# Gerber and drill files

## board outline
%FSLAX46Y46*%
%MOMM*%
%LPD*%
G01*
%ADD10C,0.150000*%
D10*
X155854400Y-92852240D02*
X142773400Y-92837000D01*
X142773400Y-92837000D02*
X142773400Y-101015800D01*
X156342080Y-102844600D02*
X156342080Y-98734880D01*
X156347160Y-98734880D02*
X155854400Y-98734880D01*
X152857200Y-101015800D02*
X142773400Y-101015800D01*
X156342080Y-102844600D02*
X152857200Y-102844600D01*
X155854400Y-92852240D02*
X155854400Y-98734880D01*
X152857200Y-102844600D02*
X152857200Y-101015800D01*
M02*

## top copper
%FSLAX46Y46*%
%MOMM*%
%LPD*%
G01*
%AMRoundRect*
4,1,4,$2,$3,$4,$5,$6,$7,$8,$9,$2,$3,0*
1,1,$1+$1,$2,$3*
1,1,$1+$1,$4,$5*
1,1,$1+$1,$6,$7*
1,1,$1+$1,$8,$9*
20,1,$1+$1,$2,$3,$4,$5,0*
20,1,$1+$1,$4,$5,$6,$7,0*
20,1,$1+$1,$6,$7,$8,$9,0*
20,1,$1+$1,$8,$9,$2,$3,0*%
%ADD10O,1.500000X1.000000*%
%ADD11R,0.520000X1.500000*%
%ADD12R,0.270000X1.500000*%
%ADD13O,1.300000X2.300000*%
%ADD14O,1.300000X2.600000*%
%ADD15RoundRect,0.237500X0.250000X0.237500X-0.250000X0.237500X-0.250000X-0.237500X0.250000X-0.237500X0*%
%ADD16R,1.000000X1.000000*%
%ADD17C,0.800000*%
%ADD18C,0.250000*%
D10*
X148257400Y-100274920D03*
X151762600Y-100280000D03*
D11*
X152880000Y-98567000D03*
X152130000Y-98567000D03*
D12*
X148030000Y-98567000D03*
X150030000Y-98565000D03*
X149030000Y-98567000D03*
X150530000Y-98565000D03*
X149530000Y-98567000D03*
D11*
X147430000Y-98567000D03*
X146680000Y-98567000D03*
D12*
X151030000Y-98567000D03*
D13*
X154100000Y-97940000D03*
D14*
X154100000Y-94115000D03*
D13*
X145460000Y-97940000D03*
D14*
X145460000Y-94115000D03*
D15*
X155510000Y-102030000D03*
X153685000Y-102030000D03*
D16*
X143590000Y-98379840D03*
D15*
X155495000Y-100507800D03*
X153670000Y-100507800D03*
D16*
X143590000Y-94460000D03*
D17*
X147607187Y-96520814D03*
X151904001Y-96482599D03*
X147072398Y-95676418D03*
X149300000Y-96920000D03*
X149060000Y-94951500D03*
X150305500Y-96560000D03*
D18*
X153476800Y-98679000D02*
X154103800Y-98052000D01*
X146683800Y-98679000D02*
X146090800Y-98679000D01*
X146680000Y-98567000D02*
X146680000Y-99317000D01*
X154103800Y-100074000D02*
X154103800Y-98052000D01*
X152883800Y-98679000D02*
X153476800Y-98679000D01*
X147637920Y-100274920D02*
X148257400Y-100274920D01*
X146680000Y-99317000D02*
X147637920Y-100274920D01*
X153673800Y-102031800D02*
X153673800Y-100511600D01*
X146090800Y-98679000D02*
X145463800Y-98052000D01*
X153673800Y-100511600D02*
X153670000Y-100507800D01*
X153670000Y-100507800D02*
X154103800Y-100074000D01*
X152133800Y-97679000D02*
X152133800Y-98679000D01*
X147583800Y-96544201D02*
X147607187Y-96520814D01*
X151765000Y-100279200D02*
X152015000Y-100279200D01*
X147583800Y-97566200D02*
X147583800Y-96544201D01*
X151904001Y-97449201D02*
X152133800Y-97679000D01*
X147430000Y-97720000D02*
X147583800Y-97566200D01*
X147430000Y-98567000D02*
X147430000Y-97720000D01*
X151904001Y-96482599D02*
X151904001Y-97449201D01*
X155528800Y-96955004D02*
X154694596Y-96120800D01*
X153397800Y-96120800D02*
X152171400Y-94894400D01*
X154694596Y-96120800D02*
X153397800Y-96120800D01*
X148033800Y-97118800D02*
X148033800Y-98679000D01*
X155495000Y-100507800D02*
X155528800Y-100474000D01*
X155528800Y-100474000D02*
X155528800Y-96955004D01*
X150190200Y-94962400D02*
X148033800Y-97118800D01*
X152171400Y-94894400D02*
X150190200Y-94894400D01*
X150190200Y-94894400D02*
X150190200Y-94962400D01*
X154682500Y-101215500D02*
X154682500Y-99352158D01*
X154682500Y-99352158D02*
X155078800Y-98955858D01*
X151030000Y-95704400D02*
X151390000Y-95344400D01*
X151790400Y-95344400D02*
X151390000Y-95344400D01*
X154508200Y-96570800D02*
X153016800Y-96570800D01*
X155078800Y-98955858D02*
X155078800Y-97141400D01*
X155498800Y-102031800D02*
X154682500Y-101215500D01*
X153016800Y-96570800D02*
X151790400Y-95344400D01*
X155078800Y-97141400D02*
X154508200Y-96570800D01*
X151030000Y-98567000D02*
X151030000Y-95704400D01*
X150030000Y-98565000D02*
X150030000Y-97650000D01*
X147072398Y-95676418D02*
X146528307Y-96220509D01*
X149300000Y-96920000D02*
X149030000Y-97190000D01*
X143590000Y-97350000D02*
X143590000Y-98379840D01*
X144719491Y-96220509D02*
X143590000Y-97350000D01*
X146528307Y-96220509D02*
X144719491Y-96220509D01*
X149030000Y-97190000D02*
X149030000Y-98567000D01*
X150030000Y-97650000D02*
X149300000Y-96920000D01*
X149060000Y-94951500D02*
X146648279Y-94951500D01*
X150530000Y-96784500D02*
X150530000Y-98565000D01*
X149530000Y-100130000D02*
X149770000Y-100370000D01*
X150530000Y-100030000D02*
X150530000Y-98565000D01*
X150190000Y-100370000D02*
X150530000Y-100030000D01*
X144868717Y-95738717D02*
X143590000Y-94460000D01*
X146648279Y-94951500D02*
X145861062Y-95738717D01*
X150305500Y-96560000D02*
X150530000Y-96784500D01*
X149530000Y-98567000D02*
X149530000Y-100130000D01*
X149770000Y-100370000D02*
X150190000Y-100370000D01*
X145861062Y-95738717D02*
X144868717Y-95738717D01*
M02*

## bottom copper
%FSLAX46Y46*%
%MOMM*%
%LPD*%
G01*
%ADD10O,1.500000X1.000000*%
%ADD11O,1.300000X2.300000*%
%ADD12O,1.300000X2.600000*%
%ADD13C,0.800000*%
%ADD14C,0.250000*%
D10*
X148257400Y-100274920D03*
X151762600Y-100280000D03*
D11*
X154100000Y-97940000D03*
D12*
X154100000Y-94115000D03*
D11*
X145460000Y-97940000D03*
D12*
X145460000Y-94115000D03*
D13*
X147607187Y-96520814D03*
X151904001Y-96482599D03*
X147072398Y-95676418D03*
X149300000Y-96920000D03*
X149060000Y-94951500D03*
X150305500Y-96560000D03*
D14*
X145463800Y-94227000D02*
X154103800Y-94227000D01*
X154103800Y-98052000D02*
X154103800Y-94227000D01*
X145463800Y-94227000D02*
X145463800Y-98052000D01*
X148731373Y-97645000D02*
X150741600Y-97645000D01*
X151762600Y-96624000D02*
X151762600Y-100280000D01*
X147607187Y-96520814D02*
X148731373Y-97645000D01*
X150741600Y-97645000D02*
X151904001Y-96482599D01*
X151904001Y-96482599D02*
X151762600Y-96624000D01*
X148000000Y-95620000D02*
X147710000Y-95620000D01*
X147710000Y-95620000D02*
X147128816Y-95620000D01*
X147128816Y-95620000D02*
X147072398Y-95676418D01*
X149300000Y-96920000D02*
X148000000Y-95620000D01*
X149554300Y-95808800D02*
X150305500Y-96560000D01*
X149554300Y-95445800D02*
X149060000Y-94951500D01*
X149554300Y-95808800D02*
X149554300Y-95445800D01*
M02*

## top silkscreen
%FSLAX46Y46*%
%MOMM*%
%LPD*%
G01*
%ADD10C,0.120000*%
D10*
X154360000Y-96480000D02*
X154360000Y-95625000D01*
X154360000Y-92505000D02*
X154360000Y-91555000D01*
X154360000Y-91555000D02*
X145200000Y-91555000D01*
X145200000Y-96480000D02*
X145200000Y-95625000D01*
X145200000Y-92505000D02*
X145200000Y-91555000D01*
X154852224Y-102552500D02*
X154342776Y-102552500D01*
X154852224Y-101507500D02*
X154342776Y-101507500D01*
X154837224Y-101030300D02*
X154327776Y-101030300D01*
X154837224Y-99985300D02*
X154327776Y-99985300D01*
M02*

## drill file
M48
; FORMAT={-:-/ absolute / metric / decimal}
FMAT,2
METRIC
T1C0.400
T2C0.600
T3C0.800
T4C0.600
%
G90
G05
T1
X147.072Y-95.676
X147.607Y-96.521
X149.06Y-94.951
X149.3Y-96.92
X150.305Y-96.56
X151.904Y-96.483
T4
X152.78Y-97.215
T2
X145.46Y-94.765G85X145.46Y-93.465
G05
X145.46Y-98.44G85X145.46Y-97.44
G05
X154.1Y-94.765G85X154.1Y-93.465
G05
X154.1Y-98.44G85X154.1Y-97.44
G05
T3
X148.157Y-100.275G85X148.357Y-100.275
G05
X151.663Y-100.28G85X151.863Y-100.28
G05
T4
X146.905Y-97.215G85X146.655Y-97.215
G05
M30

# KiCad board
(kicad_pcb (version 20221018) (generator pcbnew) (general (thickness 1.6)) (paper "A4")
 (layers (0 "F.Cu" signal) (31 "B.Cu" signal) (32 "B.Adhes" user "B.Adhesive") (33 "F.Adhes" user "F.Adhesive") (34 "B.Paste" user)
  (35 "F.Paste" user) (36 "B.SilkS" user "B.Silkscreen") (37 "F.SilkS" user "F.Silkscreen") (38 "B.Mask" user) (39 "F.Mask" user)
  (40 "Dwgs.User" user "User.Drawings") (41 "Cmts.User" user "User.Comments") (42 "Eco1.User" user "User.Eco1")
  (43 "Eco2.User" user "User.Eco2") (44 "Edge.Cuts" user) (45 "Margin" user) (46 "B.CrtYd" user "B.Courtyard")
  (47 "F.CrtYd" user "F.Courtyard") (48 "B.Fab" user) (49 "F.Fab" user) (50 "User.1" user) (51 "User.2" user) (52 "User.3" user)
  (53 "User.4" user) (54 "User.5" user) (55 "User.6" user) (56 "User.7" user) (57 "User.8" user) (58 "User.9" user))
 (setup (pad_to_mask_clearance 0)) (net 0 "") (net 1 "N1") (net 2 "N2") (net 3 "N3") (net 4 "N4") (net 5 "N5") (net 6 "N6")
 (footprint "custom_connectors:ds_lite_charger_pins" (layer "F.Cu") (at 150.01 100.28)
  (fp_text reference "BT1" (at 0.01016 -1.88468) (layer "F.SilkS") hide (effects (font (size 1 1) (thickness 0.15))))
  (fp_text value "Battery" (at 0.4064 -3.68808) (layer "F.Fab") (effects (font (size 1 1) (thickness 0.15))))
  (pad "1" thru_hole oval (at -1.7526 -0.00508 90) (size 1 1.5) (drill oval 0.8 1) (layers "*.Cu" "*.Mask") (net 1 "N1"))
  (pad "2" thru_hole oval (at 1.7526 0 90) (size 1 1.5) (drill oval 0.8 1) (layers "*.Cu" "*.Mask") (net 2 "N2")))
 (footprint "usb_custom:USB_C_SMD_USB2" (layer "F.Cu") (at 149.78 95.265 180)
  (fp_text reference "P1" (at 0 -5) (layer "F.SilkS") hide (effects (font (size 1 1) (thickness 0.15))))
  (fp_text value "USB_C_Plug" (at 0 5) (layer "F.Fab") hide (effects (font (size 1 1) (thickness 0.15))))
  (fp_line (start -4.58 -1.215) (end -4.58 -0.36) (stroke (width 0.12) (type solid)) (layer "F.SilkS"))
  (fp_line (start -4.58 2.76) (end -4.58 3.71) (stroke (width 0.12) (type solid)) (layer "F.SilkS"))
  (fp_line (start -4.58 3.71) (end 4.58 3.71) (stroke (width 0.12) (type solid)) (layer "F.SilkS"))
  (fp_line (start 4.58 -1.215) (end 4.58 -0.36) (stroke (width 0.12) (type solid)) (layer "F.SilkS"))
  (fp_line (start 4.58 2.76) (end 4.58 3.71) (stroke (width 0.12) (type solid)) (layer "F.SilkS"))
  (pad "" np_thru_hole circle (at -3 -1.95 180) (size 0.6 0.6) (drill 0.6) (layers "F&B.Cu" "*.Mask"))
  (pad "" np_thru_hole oval (at 3 -1.95 180) (size 0.85 0.6) (drill oval 0.85 0.6) (layers "F&B.Cu" "*.Mask"))
  (pad "A1" smd rect (at -3.1 -3.302 180) (size 0.52 1.5) (layers "F.Cu" "F.Paste" "F.Mask") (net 1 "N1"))
  (pad "A4" smd rect (at -2.35 -3.302 180) (size 0.52 1.5) (layers "F.Cu" "F.Paste" "F.Mask") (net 2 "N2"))
  (pad "A5" smd rect (at 1.75 -3.302 180) (size 0.27 1.5) (layers "F.Cu" "F.Paste" "F.Mask") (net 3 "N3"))
  (pad "A6" smd rect (at -0.25 -3.3 180) (size 0.27 1.5) (layers "F.Cu" "F.Paste" "F.Mask") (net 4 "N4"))
  (pad "A6" smd rect (at 0.75 -3.302 180) (size 0.27 1.5) (layers "F.Cu" "F.Paste" "F.Mask") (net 4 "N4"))
  (pad "A7" smd rect (at -0.75 -3.3 180) (size 0.27 1.5) (layers "F.Cu" "F.Paste" "F.Mask") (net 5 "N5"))
  (pad "A7" smd rect (at 0.25 -3.302 180) (size 0.27 1.5) (layers "F.Cu" "F.Paste" "F.Mask") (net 5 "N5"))
  (pad "A9" smd rect (at 2.35 -3.302 180) (size 0.52 1.5) (layers "F.Cu" "F.Paste" "F.Mask") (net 2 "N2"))
  (pad "A12" smd rect (at 3.1 -3.302 180) (size 0.52 1.5) (layers "F.Cu" "F.Paste" "F.Mask") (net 1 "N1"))
  (pad "B5" smd rect (at -1.25 -3.302 180) (size 0.27 1.5) (layers "F.Cu" "F.Paste" "F.Mask") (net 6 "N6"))
  (pad "S1" thru_hole oval (at -4.32 -2.675 180) (size 1.3 2.3) (drill oval 0.6 1.6) (layers "*.Cu" "*.Mask") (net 1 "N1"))
  (pad "S1" thru_hole oval (at -4.32 1.15 180) (size 1.3 2.6) (drill oval 0.6 1.9) (layers "*.Cu" "*.Mask") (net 1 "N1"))
  (pad "S1" thru_hole oval (at 4.32 -2.675 180) (size 1.3 2.3) (drill oval 0.6 1.6) (layers "*.Cu" "*.Mask") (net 1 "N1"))
  (pad "S1" thru_hole oval (at 4.32 1.15 180) (size 1.3 2.6) (drill oval 0.6 1.9) (layers "*.Cu" "*.Mask") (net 1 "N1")))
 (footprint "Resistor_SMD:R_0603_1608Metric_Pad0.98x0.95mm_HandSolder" (layer "F.Cu") (at 154.5975 102.03 180)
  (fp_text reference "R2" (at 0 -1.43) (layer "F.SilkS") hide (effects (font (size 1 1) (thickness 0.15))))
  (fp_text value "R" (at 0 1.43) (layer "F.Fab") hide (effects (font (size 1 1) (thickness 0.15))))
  (fp_line (start -0.254724 -0.5225) (end 0.254724 -0.5225) (stroke (width 0.12) (type solid)) (layer "F.SilkS"))
  (fp_line (start -0.254724 0.5225) (end 0.254724 0.5225) (stroke (width 0.12) (type solid)) (layer "F.SilkS"))
  (pad "1" smd roundrect (at -0.9125 0 180) (size 0.975 0.95) (layers "F.Cu" "F.Paste" "F.Mask") (roundrect_rratio 0.25) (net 6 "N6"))
  (pad "2" smd roundrect (at 0.9125 0 180) (size 0.975 0.95) (layers "F.Cu" "F.Paste" "F.Mask") (roundrect_rratio 0.25) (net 1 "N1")))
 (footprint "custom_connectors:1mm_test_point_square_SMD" (layer "F.Cu") (at 143.59 98.39)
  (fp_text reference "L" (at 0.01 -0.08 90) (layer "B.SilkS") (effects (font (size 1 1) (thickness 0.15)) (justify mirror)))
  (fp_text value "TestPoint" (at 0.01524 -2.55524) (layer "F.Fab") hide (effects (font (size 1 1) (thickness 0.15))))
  (pad "1" smd rect (at 0 -0.01016) (size 1 1) (layers "F.Cu" "F.Paste" "F.Mask") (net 4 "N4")))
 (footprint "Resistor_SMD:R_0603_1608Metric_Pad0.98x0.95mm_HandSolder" (layer "F.Cu") (at 154.5825 100.5078 180)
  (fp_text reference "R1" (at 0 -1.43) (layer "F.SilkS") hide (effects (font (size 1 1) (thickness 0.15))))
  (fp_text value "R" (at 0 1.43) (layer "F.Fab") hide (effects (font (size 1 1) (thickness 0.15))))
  (fp_line (start -0.254724 -0.5225) (end 0.254724 -0.5225) (stroke (width 0.12) (type solid)) (layer "F.SilkS"))
  (fp_line (start -0.254724 0.5225) (end 0.254724 0.5225) (stroke (width 0.12) (type solid)) (layer "F.SilkS"))
  (pad "1" smd roundrect (at -0.9125 0 180) (size 0.975 0.95) (layers "F.Cu" "F.Paste" "F.Mask") (roundrect_rratio 0.25) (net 3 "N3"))
  (pad "2" smd roundrect (at 0.9125 0 180) (size 0.975 0.95) (layers "F.Cu" "F.Paste" "F.Mask") (roundrect_rratio 0.25) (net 1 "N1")))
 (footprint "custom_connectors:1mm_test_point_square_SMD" (layer "F.Cu") (at 143.59 94.47016)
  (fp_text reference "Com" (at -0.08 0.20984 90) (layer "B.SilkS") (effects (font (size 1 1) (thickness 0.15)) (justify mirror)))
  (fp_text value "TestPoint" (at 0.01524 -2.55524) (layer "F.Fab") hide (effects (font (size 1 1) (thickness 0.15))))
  (pad "1" smd rect (at 0 -0.01016) (size 1 1) (layers "F.Cu" "F.Paste" "F.Mask") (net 5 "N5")))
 (gr_line (start 155.8544 92.85224) (end 142.7734 92.837) (stroke (width 0.15) (type solid)) (layer "Edge.Cuts"))
 (gr_line (start 142.7734 92.837) (end 142.7734 101.0158) (stroke (width 0.15) (type solid)) (layer "Edge.Cuts"))
 (gr_line (start 156.34208 102.8446) (end 156.34208 98.73488) (stroke (width 0.15) (type solid)) (layer "Edge.Cuts"))
 (gr_line (start 156.34716 98.73488) (end 155.8544 98.73488) (stroke (width 0.15) (type solid)) (layer "Edge.Cuts"))
 (gr_line (start 152.8572 101.0158) (end 142.7734 101.0158) (stroke (width 0.15) (type solid)) (layer "Edge.Cuts"))
 (gr_line (start 156.34208 102.8446) (end 152.8572 102.8446) (stroke (width 0.15) (type solid)) (layer "Edge.Cuts"))
 (gr_line (start 155.8544 92.85224) (end 155.8544 98.73488) (stroke (width 0.15) (type solid)) (layer "Edge.Cuts"))
 (gr_line (start 152.8572 102.8446) (end 152.8572 101.0158) (stroke (width 0.15) (type solid)) (layer "Edge.Cuts"))
 (segment (start 153.4768 98.679) (end 154.1038 98.052) (width 0.25) (layer "F.Cu") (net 1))
 (segment (start 146.6838 98.679) (end 146.0908 98.679) (width 0.25) (layer "F.Cu") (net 1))
 (segment (start 146.68 98.567) (end 146.68 99.317) (width 0.25) (layer "F.Cu") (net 1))
 (segment (start 154.1038 100.074) (end 154.1038 98.052) (width 0.25) (layer "F.Cu") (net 1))
 (segment (start 152.8838 98.679) (end 153.4768 98.679) (width 0.25) (layer "F.Cu") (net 1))
 (segment (start 147.63792 100.27492) (end 148.2574 100.27492) (width 0.25) (layer "F.Cu") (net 1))
 (segment (start 146.68 99.317) (end 147.63792 100.27492) (width 0.25) (layer "F.Cu") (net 1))
 (segment (start 153.6738 102.0318) (end 153.6738 100.5116) (width 0.25) (layer "F.Cu") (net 1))
 (segment (start 146.0908 98.679) (end 145.4638 98.052) (width 0.25) (layer "F.Cu") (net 1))
 (segment (start 153.6738 100.5116) (end 153.67 100.5078) (width 0.25) (layer "F.Cu") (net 1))
 (segment (start 153.67 100.5078) (end 154.1038 100.074) (width 0.25) (layer "F.Cu") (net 1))
 (segment (start 145.4638 94.227) (end 154.1038 94.227) (width 0.25) (layer "B.Cu") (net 1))
 (segment (start 154.1038 98.052) (end 154.1038 94.227) (width 0.25) (layer "B.Cu") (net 1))
 (segment (start 145.4638 94.227) (end 145.4638 98.052) (width 0.25) (layer "B.Cu") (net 1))
 (segment (start 152.1338 97.679) (end 152.1338 98.679) (width 0.25) (layer "F.Cu") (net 2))
 (segment (start 147.5838 96.544201) (end 147.607187 96.520814) (width 0.25) (layer "F.Cu") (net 2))
 (segment (start 151.765 100.2792) (end 152.015 100.2792) (width 0.25) (layer "F.Cu") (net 2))
 (segment (start 147.5838 97.5662) (end 147.5838 96.544201) (width 0.25) (layer "F.Cu") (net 2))
 (segment (start 151.904001 97.449201) (end 152.1338 97.679) (width 0.25) (layer "F.Cu") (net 2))
 (segment (start 147.43 97.72) (end 147.5838 97.5662) (width 0.25) (layer "F.Cu") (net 2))
 (segment (start 147.43 98.567) (end 147.43 97.72) (width 0.25) (layer "F.Cu") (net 2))
 (segment (start 151.904001 96.482599) (end 151.904001 97.449201) (width 0.25) (layer "F.Cu") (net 2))
 (via (at 147.607187 96.520814) (size 0.8) (drill 0.4) (layers "F.Cu" "B.Cu") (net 2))
 (via (at 151.904001 96.482599) (size 0.8) (drill 0.4) (layers "F.Cu" "B.Cu") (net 2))
 (segment (start 148.731373 97.645) (end 150.7416 97.645) (width 0.25) (layer "B.Cu") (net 2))
 (segment (start 151.7626 96.624) (end 151.7626 100.28) (width 0.25) (layer "B.Cu") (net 2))
 (segment (start 147.607187 96.520814) (end 148.731373 97.645) (width 0.25) (layer "B.Cu") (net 2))
 (segment (start 150.7416 97.645) (end 151.904001 96.482599) (width 0.25) (layer "B.Cu") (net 2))
 (segment (start 151.904001 96.482599) (end 151.7626 96.624) (width 0.25) (layer "B.Cu") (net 2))
 (segment (start 155.5288 96.955004) (end 154.694596 96.1208) (width 0.25) (layer "F.Cu") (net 3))
 (segment (start 153.3978 96.1208) (end 152.1714 94.8944) (width 0.25) (layer "F.Cu") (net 3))
 (segment (start 154.694596 96.1208) (end 153.3978 96.1208) (width 0.25) (layer "F.Cu") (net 3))
 (segment (start 148.0338 97.1188) (end 148.0338 98.679) (width 0.25) (layer "F.Cu") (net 3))
 (segment (start 155.495 100.5078) (end 155.5288 100.474) (width 0.25) (layer "F.Cu") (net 3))
 (segment (start 155.5288 100.474) (end 155.5288 96.955004) (width 0.25) (layer "F.Cu") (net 3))
 (segment (start 150.1902 94.9624) (end 148.0338 97.1188) (width 0.25) (layer "F.Cu") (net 3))
 (segment (start 152.1714 94.8944) (end 150.1902 94.8944) (width 0.25) (layer "F.Cu") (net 3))
 (segment (start 150.1902 94.8944) (end 150.1902 94.9624) (width 0.25) (layer "F.Cu") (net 3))
 (segment (start 154.6825 101.2155) (end 154.6825 99.352158) (width 0.25) (layer "F.Cu") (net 6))
 (segment (start 154.6825 99.352158) (end 155.0788 98.955858) (width 0.25) (layer "F.Cu") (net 6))
 (segment (start 151.03 95.7044) (end 151.39 95.3444) (width 0.25) (layer "F.Cu") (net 6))
 (segment (start 151.7904 95.3444) (end 151.39 95.3444) (width 0.25) (layer "F.Cu") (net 6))
 (segment (start 154.5082 96.5708) (end 153.0168 96.5708) (width 0.25) (layer "F.Cu") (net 6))
 (segment (start 155.0788 98.955858) (end 155.0788 97.1414) (width 0.25) (layer "F.Cu") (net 6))
 (segment (start 155.4988 102.0318) (end 154.6825 101.2155) (width 0.25) (layer "F.Cu") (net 6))
 (segment (start 153.0168 96.5708) (end 151.7904 95.3444) (width 0.25) (layer "F.Cu") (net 6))
 (segment (start 155.0788 97.1414) (end 154.5082 96.5708) (width 0.25) (layer "F.Cu") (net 6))
 (segment (start 151.03 98.567) (end 151.03 95.7044) (width 0.25) (layer "F.Cu") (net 6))
 (segment (start 150.03 98.565) (end 150.03 97.65) (width 0.25) (layer "F.Cu") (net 4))
 (segment (start 147.072398 95.676418) (end 146.528307 96.220509) (width 0.25) (layer "F.Cu") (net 4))
 (segment (start 149.3 96.92) (end 149.03 97.19) (width 0.25) (layer "F.Cu") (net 4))
 (segment (start 143.59 97.35) (end 143.59 98.37984) (width 0.25) (layer "F.Cu") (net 4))
 (segment (start 144.719491 96.220509) (end 143.59 97.35) (width 0.25) (layer "F.Cu") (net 4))
 (segment (start 146.528307 96.220509) (end 144.719491 96.220509) (width 0.25) (layer "F.Cu") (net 4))
 (segment (start 149.03 97.19) (end 149.03 98.567) (width 0.25) (layer "F.Cu") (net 4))
 (segment (start 150.03 97.65) (end 149.3 96.92) (width 0.25) (layer "F.Cu") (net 4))
 (via (at 147.072398 95.676418) (size 0.8) (drill 0.4) (layers "F.Cu" "B.Cu") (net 4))
 (via (at 149.3 96.92) (size 0.8) (drill 0.4) (layers "F.Cu" "B.Cu") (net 4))
 (segment (start 148 95.62) (end 147.71 95.62) (width 0.25) (layer "B.Cu") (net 4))
 (segment (start 147.71 95.62) (end 147.128816 95.62) (width 0.25) (layer "B.Cu") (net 4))
 (segment (start 147.128816 95.62) (end 147.072398 95.676418) (width 0.25) (layer "B.Cu") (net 4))
 (segment (start 149.3 96.92) (end 148 95.62) (width 0.25) (layer "B.Cu") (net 4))
 (segment (start 149.06 94.9515) (end 146.648279 94.9515) (width 0.25) (layer "F.Cu") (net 5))
 (segment (start 150.53 96.7845) (end 150.53 98.565) (width 0.25) (layer "F.Cu") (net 5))
 (segment (start 149.53 100.13) (end 149.77 100.37) (width 0.25) (layer "F.Cu") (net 5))
 (segment (start 150.53 100.03) (end 150.53 98.565) (width 0.25) (layer "F.Cu") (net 5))
 (segment (start 150.19 100.37) (end 150.53 100.03) (width 0.25) (layer "F.Cu") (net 5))
 (segment (start 144.868717 95.738717) (end 143.59 94.46) (width 0.25) (layer "F.Cu") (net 5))
 (segment (start 146.648279 94.9515) (end 145.861062 95.738717) (width 0.25) (layer "F.Cu") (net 5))
 (segment (start 150.3055 96.56) (end 150.53 96.7845) (width 0.25) (layer "F.Cu") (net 5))
 (segment (start 149.53 98.567) (end 149.53 100.13) (width 0.25) (layer "F.Cu") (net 5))
 (segment (start 149.77 100.37) (end 150.19 100.37) (width 0.25) (layer "F.Cu") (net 5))
 (segment (start 145.861062 95.738717) (end 144.868717 95.738717) (width 0.25) (layer "F.Cu") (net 5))
 (via (at 149.06 94.9515) (size 0.8) (drill 0.4) (layers "F.Cu" "B.Cu") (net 5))
 (via (at 150.3055 96.56) (size 0.8) (drill 0.4) (layers "F.Cu" "B.Cu") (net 5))
 (segment (start 149.5543 95.8088) (end 150.3055 96.56) (width 0.25) (layer "B.Cu") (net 5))
 (segment (start 149.5543 95.4458) (end 149.06 94.9515) (width 0.25) (layer "B.Cu") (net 5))
 (segment (start 149.5543 95.8088) (end 149.5543 95.4458) (width 0.25) (layer "B.Cu") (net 5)))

